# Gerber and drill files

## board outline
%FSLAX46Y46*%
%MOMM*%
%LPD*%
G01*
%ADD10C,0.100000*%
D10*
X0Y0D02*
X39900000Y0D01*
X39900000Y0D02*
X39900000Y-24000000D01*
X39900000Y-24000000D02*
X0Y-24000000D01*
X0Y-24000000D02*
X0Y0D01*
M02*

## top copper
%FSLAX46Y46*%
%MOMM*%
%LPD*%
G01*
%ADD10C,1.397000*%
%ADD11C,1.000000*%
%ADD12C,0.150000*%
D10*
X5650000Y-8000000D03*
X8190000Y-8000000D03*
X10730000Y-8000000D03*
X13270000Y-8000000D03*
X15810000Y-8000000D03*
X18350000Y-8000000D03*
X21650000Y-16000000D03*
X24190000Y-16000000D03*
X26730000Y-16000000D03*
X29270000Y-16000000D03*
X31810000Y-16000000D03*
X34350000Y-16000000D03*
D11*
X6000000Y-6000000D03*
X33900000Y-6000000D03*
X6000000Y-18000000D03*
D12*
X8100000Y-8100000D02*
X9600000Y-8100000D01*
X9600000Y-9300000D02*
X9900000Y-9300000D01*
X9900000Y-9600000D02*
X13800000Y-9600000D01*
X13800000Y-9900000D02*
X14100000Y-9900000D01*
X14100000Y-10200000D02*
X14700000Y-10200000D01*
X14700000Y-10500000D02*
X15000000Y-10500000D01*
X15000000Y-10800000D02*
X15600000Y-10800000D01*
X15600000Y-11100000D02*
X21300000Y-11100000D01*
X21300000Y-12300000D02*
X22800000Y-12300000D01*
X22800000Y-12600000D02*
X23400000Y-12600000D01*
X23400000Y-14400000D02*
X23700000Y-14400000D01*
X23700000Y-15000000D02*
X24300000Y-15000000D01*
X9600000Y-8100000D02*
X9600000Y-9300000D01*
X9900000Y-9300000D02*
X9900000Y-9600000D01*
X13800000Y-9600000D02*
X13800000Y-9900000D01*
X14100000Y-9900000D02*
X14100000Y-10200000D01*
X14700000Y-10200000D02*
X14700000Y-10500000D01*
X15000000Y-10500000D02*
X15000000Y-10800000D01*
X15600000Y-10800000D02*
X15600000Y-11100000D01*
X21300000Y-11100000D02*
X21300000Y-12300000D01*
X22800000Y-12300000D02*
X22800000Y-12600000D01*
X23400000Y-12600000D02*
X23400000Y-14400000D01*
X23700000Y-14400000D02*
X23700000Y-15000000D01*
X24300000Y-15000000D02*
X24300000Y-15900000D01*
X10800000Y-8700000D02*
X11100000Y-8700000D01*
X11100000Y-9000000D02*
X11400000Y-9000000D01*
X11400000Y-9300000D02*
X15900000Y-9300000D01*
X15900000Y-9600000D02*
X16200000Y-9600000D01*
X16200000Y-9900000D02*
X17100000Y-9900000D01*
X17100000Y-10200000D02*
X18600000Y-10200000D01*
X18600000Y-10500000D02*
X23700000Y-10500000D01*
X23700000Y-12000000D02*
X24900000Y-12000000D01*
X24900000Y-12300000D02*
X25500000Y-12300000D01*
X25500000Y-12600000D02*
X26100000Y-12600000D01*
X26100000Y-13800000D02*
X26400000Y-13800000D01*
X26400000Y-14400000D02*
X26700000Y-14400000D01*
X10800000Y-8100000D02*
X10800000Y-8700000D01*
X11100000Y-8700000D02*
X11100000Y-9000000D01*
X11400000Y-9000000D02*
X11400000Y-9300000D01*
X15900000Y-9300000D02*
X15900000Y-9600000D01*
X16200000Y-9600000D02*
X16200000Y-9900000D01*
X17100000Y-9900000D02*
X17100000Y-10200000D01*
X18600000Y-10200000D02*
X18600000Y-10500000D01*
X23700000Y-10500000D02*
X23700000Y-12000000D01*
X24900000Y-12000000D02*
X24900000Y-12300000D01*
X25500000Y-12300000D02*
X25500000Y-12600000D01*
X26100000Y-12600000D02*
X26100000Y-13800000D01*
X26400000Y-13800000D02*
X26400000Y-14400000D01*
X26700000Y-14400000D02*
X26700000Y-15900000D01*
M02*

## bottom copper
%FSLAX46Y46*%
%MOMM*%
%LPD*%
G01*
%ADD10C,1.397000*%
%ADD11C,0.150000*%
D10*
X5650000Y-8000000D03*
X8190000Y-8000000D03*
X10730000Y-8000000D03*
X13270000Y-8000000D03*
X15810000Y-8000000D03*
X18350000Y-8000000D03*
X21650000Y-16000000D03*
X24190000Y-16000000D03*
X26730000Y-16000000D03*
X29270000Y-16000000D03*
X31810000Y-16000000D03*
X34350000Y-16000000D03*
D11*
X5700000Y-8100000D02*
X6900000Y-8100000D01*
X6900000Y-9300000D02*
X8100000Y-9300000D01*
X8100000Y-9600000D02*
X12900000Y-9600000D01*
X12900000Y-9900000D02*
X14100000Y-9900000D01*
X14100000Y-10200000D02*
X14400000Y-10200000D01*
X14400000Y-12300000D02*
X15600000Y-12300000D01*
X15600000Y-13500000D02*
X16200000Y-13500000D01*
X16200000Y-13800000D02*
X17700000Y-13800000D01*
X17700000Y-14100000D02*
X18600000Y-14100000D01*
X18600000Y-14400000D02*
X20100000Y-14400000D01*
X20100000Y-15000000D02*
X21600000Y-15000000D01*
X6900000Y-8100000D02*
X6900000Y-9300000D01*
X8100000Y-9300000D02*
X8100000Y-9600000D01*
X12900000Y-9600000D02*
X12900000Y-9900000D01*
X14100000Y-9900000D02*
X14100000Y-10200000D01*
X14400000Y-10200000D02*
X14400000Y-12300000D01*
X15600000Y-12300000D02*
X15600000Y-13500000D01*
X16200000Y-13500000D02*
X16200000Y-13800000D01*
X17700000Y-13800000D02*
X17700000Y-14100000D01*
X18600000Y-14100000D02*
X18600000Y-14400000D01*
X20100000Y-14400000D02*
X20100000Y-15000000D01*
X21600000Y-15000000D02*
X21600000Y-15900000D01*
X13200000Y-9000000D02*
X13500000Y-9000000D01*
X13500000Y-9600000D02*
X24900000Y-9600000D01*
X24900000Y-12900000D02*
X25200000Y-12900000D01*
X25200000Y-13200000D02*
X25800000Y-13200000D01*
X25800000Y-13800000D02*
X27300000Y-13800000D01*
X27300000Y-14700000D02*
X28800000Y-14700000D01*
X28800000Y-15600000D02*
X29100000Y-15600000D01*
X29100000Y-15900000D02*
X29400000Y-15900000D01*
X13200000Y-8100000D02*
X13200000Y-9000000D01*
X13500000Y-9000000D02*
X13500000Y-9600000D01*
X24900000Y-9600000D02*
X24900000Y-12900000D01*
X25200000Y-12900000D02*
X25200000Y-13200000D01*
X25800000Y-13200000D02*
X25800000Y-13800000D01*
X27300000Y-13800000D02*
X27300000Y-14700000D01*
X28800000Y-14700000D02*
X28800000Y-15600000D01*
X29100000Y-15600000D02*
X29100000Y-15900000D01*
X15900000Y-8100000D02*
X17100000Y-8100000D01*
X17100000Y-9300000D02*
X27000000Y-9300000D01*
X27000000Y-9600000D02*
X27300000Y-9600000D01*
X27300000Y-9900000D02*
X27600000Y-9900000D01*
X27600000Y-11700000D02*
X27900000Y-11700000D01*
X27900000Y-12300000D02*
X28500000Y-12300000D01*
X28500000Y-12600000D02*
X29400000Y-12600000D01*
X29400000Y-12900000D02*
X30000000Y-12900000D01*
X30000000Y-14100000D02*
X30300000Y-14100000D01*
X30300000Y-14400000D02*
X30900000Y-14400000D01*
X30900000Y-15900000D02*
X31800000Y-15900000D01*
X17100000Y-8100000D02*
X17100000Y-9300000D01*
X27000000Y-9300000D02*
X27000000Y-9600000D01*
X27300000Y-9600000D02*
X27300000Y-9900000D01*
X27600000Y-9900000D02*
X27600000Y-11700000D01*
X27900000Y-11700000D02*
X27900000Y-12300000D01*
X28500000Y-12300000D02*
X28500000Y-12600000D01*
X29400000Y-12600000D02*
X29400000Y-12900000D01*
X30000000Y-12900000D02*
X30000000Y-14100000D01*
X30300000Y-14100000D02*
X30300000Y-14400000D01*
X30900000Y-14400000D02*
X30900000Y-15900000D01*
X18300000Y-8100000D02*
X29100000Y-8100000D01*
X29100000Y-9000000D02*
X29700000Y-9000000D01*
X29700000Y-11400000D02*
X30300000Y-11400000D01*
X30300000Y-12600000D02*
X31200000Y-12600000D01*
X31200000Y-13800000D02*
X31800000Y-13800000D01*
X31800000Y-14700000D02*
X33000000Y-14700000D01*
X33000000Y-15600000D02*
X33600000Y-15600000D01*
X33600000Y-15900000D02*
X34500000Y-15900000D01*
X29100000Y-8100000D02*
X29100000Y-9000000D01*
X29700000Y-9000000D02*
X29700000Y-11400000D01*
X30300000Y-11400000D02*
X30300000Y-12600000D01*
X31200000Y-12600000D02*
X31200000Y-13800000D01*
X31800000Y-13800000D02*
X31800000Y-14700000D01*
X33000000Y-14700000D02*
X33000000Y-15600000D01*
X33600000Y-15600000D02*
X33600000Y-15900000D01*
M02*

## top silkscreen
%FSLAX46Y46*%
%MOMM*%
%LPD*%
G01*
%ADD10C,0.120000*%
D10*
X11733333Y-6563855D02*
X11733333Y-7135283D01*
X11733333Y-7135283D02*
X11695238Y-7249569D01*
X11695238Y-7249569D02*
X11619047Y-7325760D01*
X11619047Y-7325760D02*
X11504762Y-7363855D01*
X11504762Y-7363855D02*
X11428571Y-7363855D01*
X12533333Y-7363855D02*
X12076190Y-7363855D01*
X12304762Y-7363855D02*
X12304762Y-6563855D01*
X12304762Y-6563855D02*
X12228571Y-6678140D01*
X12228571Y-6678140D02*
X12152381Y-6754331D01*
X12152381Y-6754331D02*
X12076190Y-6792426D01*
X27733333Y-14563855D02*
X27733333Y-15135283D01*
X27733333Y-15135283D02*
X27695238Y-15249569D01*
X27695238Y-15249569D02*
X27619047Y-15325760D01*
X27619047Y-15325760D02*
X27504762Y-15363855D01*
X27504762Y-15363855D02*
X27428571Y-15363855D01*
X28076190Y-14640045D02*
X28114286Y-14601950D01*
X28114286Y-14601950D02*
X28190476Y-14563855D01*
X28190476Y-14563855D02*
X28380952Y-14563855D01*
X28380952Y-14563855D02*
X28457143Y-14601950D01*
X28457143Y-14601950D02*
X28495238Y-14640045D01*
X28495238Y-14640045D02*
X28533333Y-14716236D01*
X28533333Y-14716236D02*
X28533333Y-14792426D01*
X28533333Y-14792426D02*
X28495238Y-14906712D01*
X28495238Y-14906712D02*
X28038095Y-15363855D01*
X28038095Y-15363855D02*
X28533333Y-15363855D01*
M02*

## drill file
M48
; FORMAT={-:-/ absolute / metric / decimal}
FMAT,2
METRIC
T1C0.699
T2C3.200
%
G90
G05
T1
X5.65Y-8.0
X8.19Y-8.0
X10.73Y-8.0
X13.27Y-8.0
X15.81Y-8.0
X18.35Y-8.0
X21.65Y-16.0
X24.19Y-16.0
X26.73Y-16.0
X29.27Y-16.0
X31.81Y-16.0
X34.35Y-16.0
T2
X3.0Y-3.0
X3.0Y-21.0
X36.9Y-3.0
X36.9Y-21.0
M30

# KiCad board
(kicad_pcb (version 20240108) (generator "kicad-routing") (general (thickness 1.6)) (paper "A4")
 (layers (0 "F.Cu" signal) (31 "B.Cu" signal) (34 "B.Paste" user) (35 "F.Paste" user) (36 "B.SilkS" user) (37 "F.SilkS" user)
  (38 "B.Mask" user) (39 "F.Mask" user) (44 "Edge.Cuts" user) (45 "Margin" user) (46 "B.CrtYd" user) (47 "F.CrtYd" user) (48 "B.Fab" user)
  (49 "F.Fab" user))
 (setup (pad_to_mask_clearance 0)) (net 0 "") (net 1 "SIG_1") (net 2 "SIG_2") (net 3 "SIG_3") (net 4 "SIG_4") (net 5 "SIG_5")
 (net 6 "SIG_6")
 (gr_line (start 0.0000 0.0000) (end 39.9000 0.0000) (layer "Edge.Cuts") (width 0.1))
 (gr_line (start 39.9000 0.0000) (end 39.9000 24.0000) (layer "Edge.Cuts") (width 0.1))
 (gr_line (start 39.9000 24.0000) (end 0.0000 24.0000) (layer "Edge.Cuts") (width 0.1))
 (gr_line (start 0.0000 24.0000) (end 0.0000 0.0000) (layer "Edge.Cuts") (width 0.1))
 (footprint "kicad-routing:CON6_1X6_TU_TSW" (layer "F.Cu") (at 12.0000 8.0000 0)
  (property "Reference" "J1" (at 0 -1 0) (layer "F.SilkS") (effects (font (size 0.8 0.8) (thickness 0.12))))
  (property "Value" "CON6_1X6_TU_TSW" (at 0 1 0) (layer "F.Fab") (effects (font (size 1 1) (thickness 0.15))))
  (pad "1" thru_hole circle (at -6.3500 0.0000) (size 1.3970 1.3970) (drill 0.6985) (layers "*.Cu") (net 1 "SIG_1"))
  (pad "2" thru_hole circle (at -3.8100 0.0000) (size 1.3970 1.3970) (drill 0.6985) (layers "*.Cu") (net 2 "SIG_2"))
  (pad "3" thru_hole circle (at -1.2700 0.0000) (size 1.3970 1.3970) (drill 0.6985) (layers "*.Cu") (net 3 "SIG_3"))
  (pad "4" thru_hole circle (at 1.2700 0.0000) (size 1.3970 1.3970) (drill 0.6985) (layers "*.Cu") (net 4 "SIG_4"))
  (pad "5" thru_hole circle (at 3.8100 0.0000) (size 1.3970 1.3970) (drill 0.6985) (layers "*.Cu") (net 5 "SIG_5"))
  (pad "6" thru_hole circle (at 6.3500 0.0000) (size 1.3970 1.3970) (drill 0.6985) (layers "*.Cu") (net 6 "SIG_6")))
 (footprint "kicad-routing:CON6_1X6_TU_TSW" (layer "F.Cu") (at 28.0000 16.0000 0)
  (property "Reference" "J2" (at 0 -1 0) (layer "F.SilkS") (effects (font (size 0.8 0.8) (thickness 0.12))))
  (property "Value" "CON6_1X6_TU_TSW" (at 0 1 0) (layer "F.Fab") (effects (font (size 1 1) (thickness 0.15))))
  (pad "1" thru_hole circle (at -6.3500 0.0000) (size 1.3970 1.3970) (drill 0.6985) (layers "*.Cu") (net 1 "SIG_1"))
  (pad "2" thru_hole circle (at -3.8100 0.0000) (size 1.3970 1.3970) (drill 0.6985) (layers "*.Cu") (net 2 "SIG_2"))
  (pad "3" thru_hole circle (at -1.2700 0.0000) (size 1.3970 1.3970) (drill 0.6985) (layers "*.Cu") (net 3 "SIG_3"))
  (pad "4" thru_hole circle (at 1.2700 0.0000) (size 1.3970 1.3970) (drill 0.6985) (layers "*.Cu") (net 4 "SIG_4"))
  (pad "5" thru_hole circle (at 3.8100 0.0000) (size 1.3970 1.3970) (drill 0.6985) (layers "*.Cu") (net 5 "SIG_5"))
  (pad "6" thru_hole circle (at 6.3500 0.0000) (size 1.3970 1.3970) (drill 0.6985) (layers "*.Cu") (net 6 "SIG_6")))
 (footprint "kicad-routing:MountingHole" (layer "F.Cu") (at 3.000 3.000)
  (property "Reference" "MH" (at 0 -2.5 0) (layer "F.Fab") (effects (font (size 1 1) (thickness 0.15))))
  (pad "" np_thru_hole circle (at 0 0) (size 3.2 3.2) (drill 3.2) (layers "*.Cu" "*.Mask")))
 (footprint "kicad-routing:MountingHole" (layer "F.Cu") (at 36.900 3.000)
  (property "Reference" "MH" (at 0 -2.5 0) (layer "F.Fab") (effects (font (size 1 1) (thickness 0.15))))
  (pad "" np_thru_hole circle (at 0 0) (size 3.2 3.2) (drill 3.2) (layers "*.Cu" "*.Mask")))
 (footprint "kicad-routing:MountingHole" (layer "F.Cu") (at 3.000 21.000)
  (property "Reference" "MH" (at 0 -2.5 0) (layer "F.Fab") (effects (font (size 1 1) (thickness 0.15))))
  (pad "" np_thru_hole circle (at 0 0) (size 3.2 3.2) (drill 3.2) (layers "*.Cu" "*.Mask")))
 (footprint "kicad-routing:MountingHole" (layer "F.Cu") (at 36.900 21.000)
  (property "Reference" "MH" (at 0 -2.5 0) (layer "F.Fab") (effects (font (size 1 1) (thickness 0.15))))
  (pad "" np_thru_hole circle (at 0 0) (size 3.2 3.2) (drill 3.2) (layers "*.Cu" "*.Mask")))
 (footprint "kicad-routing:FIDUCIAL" (layer "F.Cu") (at 6.000 6.000)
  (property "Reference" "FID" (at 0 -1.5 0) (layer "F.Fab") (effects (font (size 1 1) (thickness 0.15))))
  (pad "1" smd circle (at 0 0) (size 1 1) (layers "F.Cu" "F.Mask")))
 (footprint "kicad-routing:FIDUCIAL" (layer "F.Cu") (at 33.900 6.000)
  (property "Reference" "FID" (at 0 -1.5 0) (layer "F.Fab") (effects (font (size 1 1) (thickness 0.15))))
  (pad "1" smd circle (at 0 0) (size 1 1) (layers "F.Cu" "F.Mask")))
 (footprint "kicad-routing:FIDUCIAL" (layer "F.Cu") (at 6.000 18.000)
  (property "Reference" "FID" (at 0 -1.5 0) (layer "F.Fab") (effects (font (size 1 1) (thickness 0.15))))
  (pad "1" smd circle (at 0 0) (size 1 1) (layers "F.Cu" "F.Mask")))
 (segment (start 5.7000 8.1000) (end 6.9000 8.1000) (width 0.1500) (layer "B.Cu") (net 1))
 (segment (start 6.9000 9.3000) (end 8.1000 9.3000) (width 0.1500) (layer "B.Cu") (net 1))
 (segment (start 8.1000 9.6000) (end 12.9000 9.6000) (width 0.1500) (layer "B.Cu") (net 1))
 (segment (start 12.9000 9.9000) (end 14.1000 9.9000) (width 0.1500) (layer "B.Cu") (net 1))
 (segment (start 14.1000 10.2000) (end 14.4000 10.2000) (width 0.1500) (layer "B.Cu") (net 1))
 (segment (start 14.4000 12.3000) (end 15.6000 12.3000) (width 0.1500) (layer "B.Cu") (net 1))
 (segment (start 15.6000 13.5000) (end 16.2000 13.5000) (width 0.1500) (layer "B.Cu") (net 1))
 (segment (start 16.2000 13.8000) (end 17.7000 13.8000) (width 0.1500) (layer "B.Cu") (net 1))
 (segment (start 17.7000 14.1000) (end 18.6000 14.1000) (width 0.1500) (layer "B.Cu") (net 1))
 (segment (start 18.6000 14.4000) (end 20.1000 14.4000) (width 0.1500) (layer "B.Cu") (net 1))
 (segment (start 20.1000 15.0000) (end 21.6000 15.0000) (width 0.1500) (layer "B.Cu") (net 1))
 (segment (start 6.9000 8.1000) (end 6.9000 9.3000) (width 0.1500) (layer "B.Cu") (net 1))
 (segment (start 8.1000 9.3000) (end 8.1000 9.6000) (width 0.1500) (layer "B.Cu") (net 1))
 (segment (start 12.9000 9.6000) (end 12.9000 9.9000) (width 0.1500) (layer "B.Cu") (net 1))
 (segment (start 14.1000 9.9000) (end 14.1000 10.2000) (width 0.1500) (layer "B.Cu") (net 1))
 (segment (start 14.4000 10.2000) (end 14.4000 12.3000) (width 0.1500) (layer "B.Cu") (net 1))
 (segment (start 15.6000 12.3000) (end 15.6000 13.5000) (width 0.1500) (layer "B.Cu") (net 1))
 (segment (start 16.2000 13.5000) (end 16.2000 13.8000) (width 0.1500) (layer "B.Cu") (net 1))
 (segment (start 17.7000 13.8000) (end 17.7000 14.1000) (width 0.1500) (layer "B.Cu") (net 1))
 (segment (start 18.6000 14.1000) (end 18.6000 14.4000) (width 0.1500) (layer "B.Cu") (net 1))
 (segment (start 20.1000 14.4000) (end 20.1000 15.0000) (width 0.1500) (layer "B.Cu") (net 1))
 (segment (start 21.6000 15.0000) (end 21.6000 15.9000) (width 0.1500) (layer "B.Cu") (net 1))
 (segment (start 8.1000 8.1000) (end 9.6000 8.1000) (width 0.1500) (layer "F.Cu") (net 2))
 (segment (start 9.6000 9.3000) (end 9.9000 9.3000) (width 0.1500) (layer "F.Cu") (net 2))
 (segment (start 9.9000 9.6000) (end 13.8000 9.6000) (width 0.1500) (layer "F.Cu") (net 2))
 (segment (start 13.8000 9.9000) (end 14.1000 9.9000) (width 0.1500) (layer "F.Cu") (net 2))
 (segment (start 14.1000 10.2000) (end 14.7000 10.2000) (width 0.1500) (layer "F.Cu") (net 2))
 (segment (start 14.7000 10.5000) (end 15.0000 10.5000) (width 0.1500) (layer "F.Cu") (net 2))
 (segment (start 15.0000 10.8000) (end 15.6000 10.8000) (width 0.1500) (layer "F.Cu") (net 2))
 (segment (start 15.6000 11.1000) (end 21.3000 11.1000) (width 0.1500) (layer "F.Cu") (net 2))
 (segment (start 21.3000 12.3000) (end 22.8000 12.3000) (width 0.1500) (layer "F.Cu") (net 2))
 (segment (start 22.8000 12.6000) (end 23.4000 12.6000) (width 0.1500) (layer "F.Cu") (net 2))
 (segment (start 23.4000 14.4000) (end 23.7000 14.4000) (width 0.1500) (layer "F.Cu") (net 2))
 (segment (start 23.7000 15.0000) (end 24.3000 15.0000) (width 0.1500) (layer "F.Cu") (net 2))
 (segment (start 9.6000 8.1000) (end 9.6000 9.3000) (width 0.1500) (layer "F.Cu") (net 2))
 (segment (start 9.9000 9.3000) (end 9.9000 9.6000) (width 0.1500) (layer "F.Cu") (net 2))
 (segment (start 13.8000 9.6000) (end 13.8000 9.9000) (width 0.1500) (layer "F.Cu") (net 2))
 (segment (start 14.1000 9.9000) (end 14.1000 10.2000) (width 0.1500) (layer "F.Cu") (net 2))
 (segment (start 14.7000 10.2000) (end 14.7000 10.5000) (width 0.1500) (layer "F.Cu") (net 2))
 (segment (start 15.0000 10.5000) (end 15.0000 10.8000) (width 0.1500) (layer "F.Cu") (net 2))
 (segment (start 15.6000 10.8000) (end 15.6000 11.1000) (width 0.1500) (layer "F.Cu") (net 2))
 (segment (start 21.3000 11.1000) (end 21.3000 12.3000) (width 0.1500) (layer "F.Cu") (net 2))
 (segment (start 22.8000 12.3000) (end 22.8000 12.6000) (width 0.1500) (layer "F.Cu") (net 2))
 (segment (start 23.4000 12.6000) (end 23.4000 14.4000) (width 0.1500) (layer "F.Cu") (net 2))
 (segment (start 23.7000 14.4000) (end 23.7000 15.0000) (width 0.1500) (layer "F.Cu") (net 2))
 (segment (start 24.3000 15.0000) (end 24.3000 15.9000) (width 0.1500) (layer "F.Cu") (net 2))
 (segment (start 10.8000 8.7000) (end 11.1000 8.7000) (width 0.1500) (layer "F.Cu") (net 3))
 (segment (start 11.1000 9.0000) (end 11.4000 9.0000) (width 0.1500) (layer "F.Cu") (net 3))
 (segment (start 11.4000 9.3000) (end 15.9000 9.3000) (width 0.1500) (layer "F.Cu") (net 3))
 (segment (start 15.9000 9.6000) (end 16.2000 9.6000) (width 0.1500) (layer "F.Cu") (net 3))
 (segment (start 16.2000 9.9000) (end 17.1000 9.9000) (width 0.1500) (layer "F.Cu") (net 3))
 (segment (start 17.1000 10.2000) (end 18.6000 10.2000) (width 0.1500) (layer "F.Cu") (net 3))
 (segment (start 18.6000 10.5000) (end 23.7000 10.5000) (width 0.1500) (layer "F.Cu") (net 3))
 (segment (start 23.7000 12.0000) (end 24.9000 12.0000) (width 0.1500) (layer "F.Cu") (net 3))
 (segment (start 24.9000 12.3000) (end 25.5000 12.3000) (width 0.1500) (layer "F.Cu") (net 3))
 (segment (start 25.5000 12.6000) (end 26.1000 12.6000) (width 0.1500) (layer "F.Cu") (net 3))
 (segment (start 26.1000 13.8000) (end 26.4000 13.8000) (width 0.1500) (layer "F.Cu") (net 3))
 (segment (start 26.4000 14.4000) (end 26.7000 14.4000) (width 0.1500) (layer "F.Cu") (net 3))
 (segment (start 10.8000 8.1000) (end 10.8000 8.7000) (width 0.1500) (layer "F.Cu") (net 3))
 (segment (start 11.1000 8.7000) (end 11.1000 9.0000) (width 0.1500) (layer "F.Cu") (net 3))
 (segment (start 11.4000 9.0000) (end 11.4000 9.3000) (width 0.1500) (layer "F.Cu") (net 3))
 (segment (start 15.9000 9.3000) (end 15.9000 9.6000) (width 0.1500) (layer "F.Cu") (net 3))
 (segment (start 16.2000 9.6000) (end 16.2000 9.9000) (width 0.1500) (layer "F.Cu") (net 3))
 (segment (start 17.1000 9.9000) (end 17.1000 10.2000) (width 0.1500) (layer "F.Cu") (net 3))
 (segment (start 18.6000 10.2000) (end 18.6000 10.5000) (width 0.1500) (layer "F.Cu") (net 3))
 (segment (start 23.7000 10.5000) (end 23.7000 12.0000) (width 0.1500) (layer "F.Cu") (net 3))
 (segment (start 24.9000 12.0000) (end 24.9000 12.3000) (width 0.1500) (layer "F.Cu") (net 3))
 (segment (start 25.5000 12.3000) (end 25.5000 12.6000) (width 0.1500) (layer "F.Cu") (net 3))
 (segment (start 26.1000 12.6000) (end 26.1000 13.8000) (width 0.1500) (layer "F.Cu") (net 3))
 (segment (start 26.4000 13.8000) (end 26.4000 14.4000) (width 0.1500) (layer "F.Cu") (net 3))
 (segment (start 26.7000 14.4000) (end 26.7000 15.9000) (width 0.1500) (layer "F.Cu") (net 3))
 (segment (start 13.2000 9.0000) (end 13.5000 9.0000) (width 0.1500) (layer "B.Cu") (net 4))
 (segment (start 13.5000 9.6000) (end 24.9000 9.6000) (width 0.1500) (layer "B.Cu") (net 4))
 (segment (start 24.9000 12.9000) (end 25.2000 12.9000) (width 0.1500) (layer "B.Cu") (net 4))
 (segment (start 25.2000 13.2000) (end 25.8000 13.2000) (width 0.1500) (layer "B.Cu") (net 4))
 (segment (start 25.8000 13.8000) (end 27.3000 13.8000) (width 0.1500) (layer "B.Cu") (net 4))
 (segment (start 27.3000 14.7000) (end 28.8000 14.7000) (width 0.1500) (layer "B.Cu") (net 4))
 (segment (start 28.8000 15.6000) (end 29.1000 15.6000) (width 0.1500) (layer "B.Cu") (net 4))
 (segment (start 29.1000 15.9000) (end 29.4000 15.9000) (width 0.1500) (layer "B.Cu") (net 4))
 (segment (start 13.2000 8.1000) (end 13.2000 9.0000) (width 0.1500) (layer "B.Cu") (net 4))
 (segment (start 13.5000 9.0000) (end 13.5000 9.6000) (width 0.1500) (layer "B.Cu") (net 4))
 (segment (start 24.9000 9.6000) (end 24.9000 12.9000) (width 0.1500) (layer "B.Cu") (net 4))
 (segment (start 25.2000 12.9000) (end 25.2000 13.2000) (width 0.1500) (layer "B.Cu") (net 4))
 (segment (start 25.8000 13.2000) (end 25.8000 13.8000) (width 0.1500) (layer "B.Cu") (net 4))
 (segment (start 27.3000 13.8000) (end 27.3000 14.7000) (width 0.1500) (layer "B.Cu") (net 4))
 (segment (start 28.8000 14.7000) (end 28.8000 15.6000) (width 0.1500) (layer "B.Cu") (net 4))
 (segment (start 29.1000 15.6000) (end 29.1000 15.9000) (width 0.1500) (layer "B.Cu") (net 4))
 (segment (start 15.9000 8.1000) (end 17.1000 8.1000) (width 0.1500) (layer "B.Cu") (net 5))
 (segment (start 17.1000 9.3000) (end 27.0000 9.3000) (width 0.1500) (layer "B.Cu") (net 5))
 (segment (start 27.0000 9.6000) (end 27.3000 9.6000) (width 0.1500) (layer "B.Cu") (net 5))
 (segment (start 27.3000 9.9000) (end 27.6000 9.9000) (width 0.1500) (layer "B.Cu") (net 5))
 (segment (start 27.6000 11.7000) (end 27.9000 11.7000) (width 0.1500) (layer "B.Cu") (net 5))
 (segment (start 27.9000 12.3000) (end 28.5000 12.3000) (width 0.1500) (layer "B.Cu") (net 5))
 (segment (start 28.5000 12.6000) (end 29.4000 12.6000) (width 0.1500) (layer "B.Cu") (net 5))
 (segment (start 29.4000 12.9000) (end 30.0000 12.9000) (width 0.1500) (layer "B.Cu") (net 5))
 (segment (start 30.0000 14.1000) (end 30.3000 14.1000) (width 0.1500) (layer "B.Cu") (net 5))
 (segment (start 30.3000 14.4000) (end 30.9000 14.4000) (width 0.1500) (layer "B.Cu") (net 5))
 (segment (start 30.9000 15.9000) (end 31.8000 15.9000) (width 0.1500) (layer "B.Cu") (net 5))
 (segment (start 17.1000 8.1000) (end 17.1000 9.3000) (width 0.1500) (layer "B.Cu") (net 5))
 (segment (start 27.0000 9.3000) (end 27.0000 9.6000) (width 0.1500) (layer "B.Cu") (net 5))
 (segment (start 27.3000 9.6000) (end 27.3000 9.9000) (width 0.1500) (layer "B.Cu") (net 5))
 (segment (start 27.6000 9.9000) (end 27.6000 11.7000) (width 0.1500) (layer "B.Cu") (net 5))
 (segment (start 27.9000 11.7000) (end 27.9000 12.3000) (width 0.1500) (layer "B.Cu") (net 5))
 (segment (start 28.5000 12.3000) (end 28.5000 12.6000) (width 0.1500) (layer "B.Cu") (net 5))
 (segment (start 29.4000 12.6000) (end 29.4000 12.9000) (width 0.1500) (layer "B.Cu") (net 5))
 (segment (start 30.0000 12.9000) (end 30.0000 14.1000) (width 0.1500) (layer "B.Cu") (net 5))
 (segment (start 30.3000 14.1000) (end 30.3000 14.4000) (width 0.1500) (layer "B.Cu") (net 5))
 (segment (start 30.9000 14.4000) (end 30.9000 15.9000) (width 0.1500) (layer "B.Cu") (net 5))
 (segment (start 18.3000 8.1000) (end 29.1000 8.1000) (width 0.1500) (layer "B.Cu") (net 6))
 (segment (start 29.1000 9.0000) (end 29.7000 9.0000) (width 0.1500) (layer "B.Cu") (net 6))
 (segment (start 29.7000 11.4000) (end 30.3000 11.4000) (width 0.1500) (layer "B.Cu") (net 6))
 (segment (start 30.3000 12.6000) (end 31.2000 12.6000) (width 0.1500) (layer "B.Cu") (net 6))
 (segment (start 31.2000 13.8000) (end 31.8000 13.8000) (width 0.1500) (layer "B.Cu") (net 6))
 (segment (start 31.8000 14.7000) (end 33.0000 14.7000) (width 0.1500) (layer "B.Cu") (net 6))
 (segment (start 33.0000 15.6000) (end 33.6000 15.6000) (width 0.1500) (layer "B.Cu") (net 6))
 (segment (start 33.6000 15.9000) (end 34.5000 15.9000) (width 0.1500) (layer "B.Cu") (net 6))
 (segment (start 29.1000 8.1000) (end 29.1000 9.0000) (width 0.1500) (layer "B.Cu") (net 6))
 (segment (start 29.7000 9.0000) (end 29.7000 11.4000) (width 0.1500) (layer "B.Cu") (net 6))
 (segment (start 30.3000 11.4000) (end 30.3000 12.6000) (width 0.1500) (layer "B.Cu") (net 6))
 (segment (start 31.2000 12.6000) (end 31.2000 13.8000) (width 0.1500) (layer "B.Cu") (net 6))
 (segment (start 31.8000 13.8000) (end 31.8000 14.7000) (width 0.1500) (layer "B.Cu") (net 6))
 (segment (start 33.0000 14.7000) (end 33.0000 15.6000) (width 0.1500) (layer "B.Cu") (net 6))
 (segment (start 33.6000 15.6000) (end 33.6000 15.9000) (width 0.1500) (layer "B.Cu") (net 6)))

